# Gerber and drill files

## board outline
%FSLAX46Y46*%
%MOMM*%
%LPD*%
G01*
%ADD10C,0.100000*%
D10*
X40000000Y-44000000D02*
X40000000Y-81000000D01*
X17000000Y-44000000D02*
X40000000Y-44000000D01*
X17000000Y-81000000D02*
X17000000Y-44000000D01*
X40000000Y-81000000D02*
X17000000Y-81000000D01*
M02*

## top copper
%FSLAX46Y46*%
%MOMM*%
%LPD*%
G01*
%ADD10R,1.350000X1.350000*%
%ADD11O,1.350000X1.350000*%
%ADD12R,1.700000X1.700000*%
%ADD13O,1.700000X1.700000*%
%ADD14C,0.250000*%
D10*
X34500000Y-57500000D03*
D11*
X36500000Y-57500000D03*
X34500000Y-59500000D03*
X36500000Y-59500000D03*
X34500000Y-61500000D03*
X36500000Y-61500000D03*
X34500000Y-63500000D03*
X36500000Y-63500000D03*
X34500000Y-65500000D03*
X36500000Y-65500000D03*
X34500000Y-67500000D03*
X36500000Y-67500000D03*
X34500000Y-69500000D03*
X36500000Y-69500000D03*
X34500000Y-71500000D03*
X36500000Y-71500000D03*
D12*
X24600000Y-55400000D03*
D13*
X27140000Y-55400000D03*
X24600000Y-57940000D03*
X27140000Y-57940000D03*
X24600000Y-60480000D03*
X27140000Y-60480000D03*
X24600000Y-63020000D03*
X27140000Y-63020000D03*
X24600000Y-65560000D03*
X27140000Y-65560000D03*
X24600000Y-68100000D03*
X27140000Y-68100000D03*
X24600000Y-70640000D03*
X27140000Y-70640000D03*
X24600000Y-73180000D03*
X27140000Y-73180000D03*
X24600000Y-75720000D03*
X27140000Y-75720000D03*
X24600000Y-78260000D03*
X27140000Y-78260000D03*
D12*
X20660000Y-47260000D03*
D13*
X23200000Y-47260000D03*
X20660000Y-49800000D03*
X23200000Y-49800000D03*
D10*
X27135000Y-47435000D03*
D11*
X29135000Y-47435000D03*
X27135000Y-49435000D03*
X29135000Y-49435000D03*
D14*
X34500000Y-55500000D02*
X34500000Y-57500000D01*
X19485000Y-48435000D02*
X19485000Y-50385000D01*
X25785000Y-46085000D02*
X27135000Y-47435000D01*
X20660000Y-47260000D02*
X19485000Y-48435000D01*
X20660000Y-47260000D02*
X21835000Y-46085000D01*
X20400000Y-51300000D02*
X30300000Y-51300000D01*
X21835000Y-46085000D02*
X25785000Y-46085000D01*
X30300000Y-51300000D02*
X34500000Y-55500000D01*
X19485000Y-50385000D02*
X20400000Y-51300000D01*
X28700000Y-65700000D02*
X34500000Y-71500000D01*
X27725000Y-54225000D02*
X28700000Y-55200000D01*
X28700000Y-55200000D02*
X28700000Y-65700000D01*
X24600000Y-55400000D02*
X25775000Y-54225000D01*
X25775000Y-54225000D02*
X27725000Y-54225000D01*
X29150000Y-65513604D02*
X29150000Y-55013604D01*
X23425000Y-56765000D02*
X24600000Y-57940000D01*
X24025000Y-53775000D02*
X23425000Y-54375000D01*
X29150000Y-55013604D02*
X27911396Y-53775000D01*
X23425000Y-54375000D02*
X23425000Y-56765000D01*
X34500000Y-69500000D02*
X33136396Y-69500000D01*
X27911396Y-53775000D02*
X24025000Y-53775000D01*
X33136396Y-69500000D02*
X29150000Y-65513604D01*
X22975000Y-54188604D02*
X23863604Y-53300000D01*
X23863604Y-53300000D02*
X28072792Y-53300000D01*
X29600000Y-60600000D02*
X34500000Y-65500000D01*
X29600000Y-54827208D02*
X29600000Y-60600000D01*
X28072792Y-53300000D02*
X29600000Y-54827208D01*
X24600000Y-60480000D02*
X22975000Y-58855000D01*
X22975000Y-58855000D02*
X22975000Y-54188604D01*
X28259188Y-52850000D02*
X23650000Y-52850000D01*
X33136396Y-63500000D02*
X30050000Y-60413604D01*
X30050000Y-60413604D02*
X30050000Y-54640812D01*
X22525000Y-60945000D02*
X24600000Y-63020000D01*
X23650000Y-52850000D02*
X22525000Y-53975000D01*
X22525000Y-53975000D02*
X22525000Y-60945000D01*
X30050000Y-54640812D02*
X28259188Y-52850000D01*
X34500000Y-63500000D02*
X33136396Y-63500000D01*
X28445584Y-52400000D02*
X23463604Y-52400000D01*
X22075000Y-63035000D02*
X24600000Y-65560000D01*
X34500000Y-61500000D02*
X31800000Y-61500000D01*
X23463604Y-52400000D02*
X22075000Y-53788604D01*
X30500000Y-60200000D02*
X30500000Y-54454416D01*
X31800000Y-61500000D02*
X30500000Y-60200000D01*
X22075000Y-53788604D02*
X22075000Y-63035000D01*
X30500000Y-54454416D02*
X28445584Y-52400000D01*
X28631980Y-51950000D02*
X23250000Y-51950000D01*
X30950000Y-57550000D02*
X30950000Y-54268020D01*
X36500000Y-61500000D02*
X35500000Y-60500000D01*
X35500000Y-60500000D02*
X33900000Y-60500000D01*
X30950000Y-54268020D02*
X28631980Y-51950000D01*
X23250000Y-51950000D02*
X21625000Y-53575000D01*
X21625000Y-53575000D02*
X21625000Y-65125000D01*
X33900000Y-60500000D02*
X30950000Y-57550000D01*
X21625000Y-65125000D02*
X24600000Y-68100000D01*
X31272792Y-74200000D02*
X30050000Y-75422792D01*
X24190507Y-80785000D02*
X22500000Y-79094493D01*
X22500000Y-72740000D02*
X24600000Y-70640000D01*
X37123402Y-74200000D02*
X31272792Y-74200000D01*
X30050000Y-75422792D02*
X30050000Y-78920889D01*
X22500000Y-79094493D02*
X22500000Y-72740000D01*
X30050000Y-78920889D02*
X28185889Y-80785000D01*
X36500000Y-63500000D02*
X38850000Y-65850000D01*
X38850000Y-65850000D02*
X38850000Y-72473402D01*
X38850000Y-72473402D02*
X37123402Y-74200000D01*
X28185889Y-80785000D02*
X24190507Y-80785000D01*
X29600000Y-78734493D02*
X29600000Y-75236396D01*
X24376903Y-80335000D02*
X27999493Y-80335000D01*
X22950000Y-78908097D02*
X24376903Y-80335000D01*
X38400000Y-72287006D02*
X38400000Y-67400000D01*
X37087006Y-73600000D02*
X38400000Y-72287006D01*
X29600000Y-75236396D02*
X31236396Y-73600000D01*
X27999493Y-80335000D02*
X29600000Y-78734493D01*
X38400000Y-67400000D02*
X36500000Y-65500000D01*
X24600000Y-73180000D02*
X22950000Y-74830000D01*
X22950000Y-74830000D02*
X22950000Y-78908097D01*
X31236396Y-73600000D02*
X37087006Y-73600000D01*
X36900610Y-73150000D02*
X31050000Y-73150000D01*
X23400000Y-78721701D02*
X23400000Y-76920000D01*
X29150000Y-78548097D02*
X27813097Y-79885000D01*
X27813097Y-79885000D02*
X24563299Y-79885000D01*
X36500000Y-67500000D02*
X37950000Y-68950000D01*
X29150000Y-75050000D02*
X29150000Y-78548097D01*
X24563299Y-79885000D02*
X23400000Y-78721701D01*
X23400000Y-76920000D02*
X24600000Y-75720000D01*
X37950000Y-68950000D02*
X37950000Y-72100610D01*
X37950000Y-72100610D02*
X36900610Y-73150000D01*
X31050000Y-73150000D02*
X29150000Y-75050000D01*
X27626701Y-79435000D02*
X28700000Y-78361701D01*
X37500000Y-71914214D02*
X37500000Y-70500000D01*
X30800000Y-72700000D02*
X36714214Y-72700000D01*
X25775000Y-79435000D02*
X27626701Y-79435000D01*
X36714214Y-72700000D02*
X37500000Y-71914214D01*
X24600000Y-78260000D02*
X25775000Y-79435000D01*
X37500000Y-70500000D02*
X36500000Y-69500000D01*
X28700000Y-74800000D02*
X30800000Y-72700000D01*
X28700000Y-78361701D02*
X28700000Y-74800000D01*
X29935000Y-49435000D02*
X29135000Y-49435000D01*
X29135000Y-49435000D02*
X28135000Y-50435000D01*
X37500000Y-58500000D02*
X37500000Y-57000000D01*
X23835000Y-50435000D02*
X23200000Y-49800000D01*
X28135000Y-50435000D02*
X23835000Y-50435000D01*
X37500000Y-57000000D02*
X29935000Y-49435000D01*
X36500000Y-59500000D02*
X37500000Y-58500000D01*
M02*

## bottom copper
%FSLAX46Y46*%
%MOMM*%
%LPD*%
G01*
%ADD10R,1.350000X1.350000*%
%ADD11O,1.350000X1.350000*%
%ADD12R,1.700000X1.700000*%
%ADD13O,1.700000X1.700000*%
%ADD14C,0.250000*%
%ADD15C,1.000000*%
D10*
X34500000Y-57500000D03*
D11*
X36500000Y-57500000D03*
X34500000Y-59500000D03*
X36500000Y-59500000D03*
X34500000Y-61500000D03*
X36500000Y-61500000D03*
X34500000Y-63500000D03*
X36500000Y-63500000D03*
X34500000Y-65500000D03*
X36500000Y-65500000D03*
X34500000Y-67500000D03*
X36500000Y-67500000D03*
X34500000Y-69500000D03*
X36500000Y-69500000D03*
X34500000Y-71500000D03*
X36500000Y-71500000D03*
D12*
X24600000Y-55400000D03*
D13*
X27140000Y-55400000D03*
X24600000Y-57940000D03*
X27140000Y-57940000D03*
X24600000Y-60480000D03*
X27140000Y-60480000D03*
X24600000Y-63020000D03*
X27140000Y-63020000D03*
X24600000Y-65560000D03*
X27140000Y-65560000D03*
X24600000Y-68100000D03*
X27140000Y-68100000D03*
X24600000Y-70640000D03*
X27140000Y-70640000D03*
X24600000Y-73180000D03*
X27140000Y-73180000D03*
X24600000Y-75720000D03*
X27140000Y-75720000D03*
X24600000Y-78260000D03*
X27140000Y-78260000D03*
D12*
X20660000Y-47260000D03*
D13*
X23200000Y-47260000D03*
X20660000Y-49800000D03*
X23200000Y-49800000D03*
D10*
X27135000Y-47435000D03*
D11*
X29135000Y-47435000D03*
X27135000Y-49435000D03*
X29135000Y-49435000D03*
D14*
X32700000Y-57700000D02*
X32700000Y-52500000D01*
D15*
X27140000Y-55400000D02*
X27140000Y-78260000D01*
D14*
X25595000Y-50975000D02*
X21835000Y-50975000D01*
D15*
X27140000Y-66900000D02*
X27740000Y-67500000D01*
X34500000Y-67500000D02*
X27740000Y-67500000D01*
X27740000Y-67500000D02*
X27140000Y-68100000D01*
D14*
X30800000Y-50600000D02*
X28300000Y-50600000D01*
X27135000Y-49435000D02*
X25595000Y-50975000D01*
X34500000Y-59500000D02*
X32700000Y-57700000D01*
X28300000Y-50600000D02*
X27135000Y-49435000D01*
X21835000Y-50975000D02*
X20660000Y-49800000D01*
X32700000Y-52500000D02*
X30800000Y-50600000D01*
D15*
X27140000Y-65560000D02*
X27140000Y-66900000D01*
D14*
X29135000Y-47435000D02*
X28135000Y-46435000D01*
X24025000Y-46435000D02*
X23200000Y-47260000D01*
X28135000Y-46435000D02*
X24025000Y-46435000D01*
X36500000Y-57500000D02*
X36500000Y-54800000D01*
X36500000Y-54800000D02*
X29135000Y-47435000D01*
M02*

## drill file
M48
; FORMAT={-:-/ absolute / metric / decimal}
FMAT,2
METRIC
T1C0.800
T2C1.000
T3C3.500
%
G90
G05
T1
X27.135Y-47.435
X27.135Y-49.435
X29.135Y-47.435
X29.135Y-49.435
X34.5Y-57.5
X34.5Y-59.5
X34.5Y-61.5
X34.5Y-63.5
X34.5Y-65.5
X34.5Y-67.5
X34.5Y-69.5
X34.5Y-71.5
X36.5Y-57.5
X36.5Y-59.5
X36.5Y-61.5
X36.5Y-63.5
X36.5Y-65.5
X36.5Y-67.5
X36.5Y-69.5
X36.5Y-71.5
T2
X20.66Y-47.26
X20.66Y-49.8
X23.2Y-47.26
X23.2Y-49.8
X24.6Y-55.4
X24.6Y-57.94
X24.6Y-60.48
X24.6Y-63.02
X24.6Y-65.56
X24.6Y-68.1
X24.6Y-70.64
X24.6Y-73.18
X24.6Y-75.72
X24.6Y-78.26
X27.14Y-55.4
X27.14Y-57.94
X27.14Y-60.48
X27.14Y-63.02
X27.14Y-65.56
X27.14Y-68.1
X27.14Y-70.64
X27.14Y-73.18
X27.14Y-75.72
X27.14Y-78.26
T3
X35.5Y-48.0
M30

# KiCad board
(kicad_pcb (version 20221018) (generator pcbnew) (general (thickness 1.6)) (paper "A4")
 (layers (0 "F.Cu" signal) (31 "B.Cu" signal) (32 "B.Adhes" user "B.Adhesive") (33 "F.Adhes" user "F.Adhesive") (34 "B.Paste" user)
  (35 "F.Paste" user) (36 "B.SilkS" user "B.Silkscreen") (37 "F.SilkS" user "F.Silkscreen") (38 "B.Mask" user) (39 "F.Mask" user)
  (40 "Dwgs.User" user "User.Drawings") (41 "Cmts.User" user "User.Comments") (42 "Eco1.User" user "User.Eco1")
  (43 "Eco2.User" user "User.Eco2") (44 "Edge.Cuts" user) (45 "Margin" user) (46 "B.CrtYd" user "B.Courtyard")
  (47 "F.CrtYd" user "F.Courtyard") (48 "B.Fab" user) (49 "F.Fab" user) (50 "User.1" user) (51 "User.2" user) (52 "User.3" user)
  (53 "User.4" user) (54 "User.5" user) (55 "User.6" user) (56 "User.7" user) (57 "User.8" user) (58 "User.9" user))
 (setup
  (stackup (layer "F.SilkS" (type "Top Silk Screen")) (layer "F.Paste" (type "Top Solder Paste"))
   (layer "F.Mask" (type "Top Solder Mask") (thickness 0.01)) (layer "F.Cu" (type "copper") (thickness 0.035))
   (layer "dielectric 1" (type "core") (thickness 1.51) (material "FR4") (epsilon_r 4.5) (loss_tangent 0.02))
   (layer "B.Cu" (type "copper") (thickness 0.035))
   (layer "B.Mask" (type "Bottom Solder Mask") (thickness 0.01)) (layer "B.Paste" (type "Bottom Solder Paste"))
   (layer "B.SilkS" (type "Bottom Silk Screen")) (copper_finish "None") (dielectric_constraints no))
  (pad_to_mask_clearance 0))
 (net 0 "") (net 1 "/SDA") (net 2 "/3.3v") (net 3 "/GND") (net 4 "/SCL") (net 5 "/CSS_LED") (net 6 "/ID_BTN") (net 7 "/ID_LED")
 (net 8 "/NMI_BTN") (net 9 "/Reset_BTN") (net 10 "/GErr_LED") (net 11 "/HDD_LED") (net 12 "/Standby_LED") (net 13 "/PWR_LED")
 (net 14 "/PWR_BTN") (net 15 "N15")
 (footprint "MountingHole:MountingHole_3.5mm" (layer "F.Cu") (at 35.5 48)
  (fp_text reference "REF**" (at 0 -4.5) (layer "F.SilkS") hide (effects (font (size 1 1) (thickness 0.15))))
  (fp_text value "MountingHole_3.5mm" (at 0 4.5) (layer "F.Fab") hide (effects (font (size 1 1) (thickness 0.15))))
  (pad "" np_thru_hole circle (at 0 0) (size 3.5 3.5) (drill 3.5) (layers "*.Cu" "*.Mask")))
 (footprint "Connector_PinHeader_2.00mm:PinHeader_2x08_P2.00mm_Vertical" (layer "F.Cu") (at 34.5 57.5)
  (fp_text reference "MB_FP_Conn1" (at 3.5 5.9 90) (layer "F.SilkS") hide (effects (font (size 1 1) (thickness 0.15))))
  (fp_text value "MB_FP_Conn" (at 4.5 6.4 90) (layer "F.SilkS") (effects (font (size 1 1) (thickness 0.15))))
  (pad "1" thru_hole rect (at 0 0) (size 1.35 1.35) (drill 0.8) (layers "*.Cu" "*.Mask") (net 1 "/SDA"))
  (pad "2" thru_hole oval (at 2 0) (size 1.35 1.35) (drill 0.8) (layers "*.Cu" "*.Mask") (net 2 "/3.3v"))
  (pad "3" thru_hole oval (at 0 2) (size 1.35 1.35) (drill 0.8) (layers "*.Cu" "*.Mask") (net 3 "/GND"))
  (pad "4" thru_hole oval (at 2 2) (size 1.35 1.35) (drill 0.8) (layers "*.Cu" "*.Mask") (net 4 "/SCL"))
  (pad "5" thru_hole oval (at 0 4) (size 1.35 1.35) (drill 0.8) (layers "*.Cu" "*.Mask") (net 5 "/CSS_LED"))
  (pad "6" thru_hole oval (at 2 4) (size 1.35 1.35) (drill 0.8) (layers "*.Cu" "*.Mask") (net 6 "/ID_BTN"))
  (pad "7" thru_hole oval (at 0 6) (size 1.35 1.35) (drill 0.8) (layers "*.Cu" "*.Mask") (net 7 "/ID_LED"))
  (pad "8" thru_hole oval (at 2 6) (size 1.35 1.35) (drill 0.8) (layers "*.Cu" "*.Mask") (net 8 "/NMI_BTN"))
  (pad "9" thru_hole oval (at 0 8) (size 1.35 1.35) (drill 0.8) (layers "*.Cu" "*.Mask") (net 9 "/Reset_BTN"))
  (pad "10" thru_hole oval (at 2 8) (size 1.35 1.35) (drill 0.8) (layers "*.Cu" "*.Mask") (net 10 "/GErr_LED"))
  (pad "11" thru_hole oval (at 0 10) (size 1.35 1.35) (drill 0.8) (layers "*.Cu" "*.Mask") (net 3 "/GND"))
  (pad "12" thru_hole oval (at 2 10) (size 1.35 1.35) (drill 0.8) (layers "*.Cu" "*.Mask") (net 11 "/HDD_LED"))
  (pad "13" thru_hole oval (at 0 12) (size 1.35 1.35) (drill 0.8) (layers "*.Cu" "*.Mask") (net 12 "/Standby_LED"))
  (pad "14" thru_hole oval (at 2 12) (size 1.35 1.35) (drill 0.8) (layers "*.Cu" "*.Mask") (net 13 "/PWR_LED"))
  (pad "15" thru_hole oval (at 0 14) (size 1.35 1.35) (drill 0.8) (layers "*.Cu" "*.Mask") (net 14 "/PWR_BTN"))
  (pad "16" thru_hole oval (at 2 14) (size 1.35 1.35) (drill 0.8) (layers "*.Cu" "*.Mask") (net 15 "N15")))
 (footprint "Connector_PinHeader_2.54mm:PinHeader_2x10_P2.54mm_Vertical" (layer "F.Cu") (at 24.6 55.4)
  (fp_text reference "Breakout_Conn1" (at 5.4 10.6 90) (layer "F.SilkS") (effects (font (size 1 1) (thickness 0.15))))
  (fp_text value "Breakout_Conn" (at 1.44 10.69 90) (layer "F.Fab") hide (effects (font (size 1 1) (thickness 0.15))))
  (pad "1" thru_hole rect (at 0 0) (size 1.7 1.7) (drill 1) (layers "*.Cu" "*.Mask") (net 14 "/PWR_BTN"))
  (pad "2" thru_hole oval (at 2.54 0) (size 1.7 1.7) (drill 1) (layers "*.Cu" "*.Mask") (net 3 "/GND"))
  (pad "3" thru_hole oval (at 0 2.54) (size 1.7 1.7) (drill 1) (layers "*.Cu" "*.Mask") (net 12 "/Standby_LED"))
  (pad "4" thru_hole oval (at 2.54 2.54) (size 1.7 1.7) (drill 1) (layers "*.Cu" "*.Mask") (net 3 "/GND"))
  (pad "5" thru_hole oval (at 0 5.08) (size 1.7 1.7) (drill 1) (layers "*.Cu" "*.Mask") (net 9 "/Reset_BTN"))
  (pad "6" thru_hole oval (at 2.54 5.08) (size 1.7 1.7) (drill 1) (layers "*.Cu" "*.Mask") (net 3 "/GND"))
  (pad "7" thru_hole oval (at 0 7.62) (size 1.7 1.7) (drill 1) (layers "*.Cu" "*.Mask") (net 7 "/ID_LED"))
  (pad "8" thru_hole oval (at 2.54 7.62) (size 1.7 1.7) (drill 1) (layers "*.Cu" "*.Mask") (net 3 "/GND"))
  (pad "9" thru_hole oval (at 0 10.16) (size 1.7 1.7) (drill 1) (layers "*.Cu" "*.Mask") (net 5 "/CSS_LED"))
  (pad "10" thru_hole oval (at 2.54 10.16) (size 1.7 1.7) (drill 1) (layers "*.Cu" "*.Mask") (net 3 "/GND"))
  (pad "11" thru_hole oval (at 0 12.7) (size 1.7 1.7) (drill 1) (layers "*.Cu" "*.Mask") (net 6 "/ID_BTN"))
  (pad "12" thru_hole oval (at 2.54 12.7) (size 1.7 1.7) (drill 1) (layers "*.Cu" "*.Mask") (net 3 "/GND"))
  (pad "13" thru_hole oval (at 0 15.24) (size 1.7 1.7) (drill 1) (layers "*.Cu" "*.Mask") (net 8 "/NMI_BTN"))
  (pad "14" thru_hole oval (at 2.54 15.24) (size 1.7 1.7) (drill 1) (layers "*.Cu" "*.Mask") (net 3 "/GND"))
  (pad "15" thru_hole oval (at 0 17.78) (size 1.7 1.7) (drill 1) (layers "*.Cu" "*.Mask") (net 10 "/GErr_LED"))
  (pad "16" thru_hole oval (at 2.54 17.78) (size 1.7 1.7) (drill 1) (layers "*.Cu" "*.Mask") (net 3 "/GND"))
  (pad "17" thru_hole oval (at 0 20.32) (size 1.7 1.7) (drill 1) (layers "*.Cu" "*.Mask") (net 11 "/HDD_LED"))
  (pad "18" thru_hole oval (at 2.54 20.32) (size 1.7 1.7) (drill 1) (layers "*.Cu" "*.Mask") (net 3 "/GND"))
  (pad "19" thru_hole oval (at 0 22.86) (size 1.7 1.7) (drill 1) (layers "*.Cu" "*.Mask") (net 13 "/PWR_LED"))
  (pad "20" thru_hole oval (at 2.54 22.86) (size 1.7 1.7) (drill 1) (layers "*.Cu" "*.Mask") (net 3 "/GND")))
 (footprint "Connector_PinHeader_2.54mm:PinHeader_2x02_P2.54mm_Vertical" (layer "F.Cu") (at 20.66 47.26)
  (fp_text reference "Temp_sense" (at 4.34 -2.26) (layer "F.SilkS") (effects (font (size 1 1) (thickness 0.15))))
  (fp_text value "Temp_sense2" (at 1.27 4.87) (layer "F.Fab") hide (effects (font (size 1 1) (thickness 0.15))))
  (pad "1" thru_hole rect (at 0 0) (size 1.7 1.7) (drill 1) (layers "*.Cu" "*.Mask") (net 1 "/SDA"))
  (pad "2" thru_hole oval (at 2.54 0) (size 1.7 1.7) (drill 1) (layers "*.Cu" "*.Mask") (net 2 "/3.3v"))
  (pad "3" thru_hole oval (at 0 2.54) (size 1.7 1.7) (drill 1) (layers "*.Cu" "*.Mask") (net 3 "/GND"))
  (pad "4" thru_hole oval (at 2.54 2.54) (size 1.7 1.7) (drill 1) (layers "*.Cu" "*.Mask") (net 4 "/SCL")))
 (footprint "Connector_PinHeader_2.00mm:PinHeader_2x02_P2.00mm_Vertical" (layer "F.Cu") (at 27.135 47.435)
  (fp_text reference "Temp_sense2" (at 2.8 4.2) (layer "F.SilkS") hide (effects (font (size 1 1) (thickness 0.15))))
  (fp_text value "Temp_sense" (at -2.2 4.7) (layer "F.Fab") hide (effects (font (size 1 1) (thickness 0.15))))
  (pad "1" thru_hole rect (at 0 0) (size 1.35 1.35) (drill 0.8) (layers "*.Cu" "*.Mask") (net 1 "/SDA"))
  (pad "2" thru_hole oval (at 2 0) (size 1.35 1.35) (drill 0.8) (layers "*.Cu" "*.Mask") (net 2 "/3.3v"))
  (pad "3" thru_hole oval (at 0 2) (size 1.35 1.35) (drill 0.8) (layers "*.Cu" "*.Mask") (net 3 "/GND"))
  (pad "4" thru_hole oval (at 2 2) (size 1.35 1.35) (drill 0.8) (layers "*.Cu" "*.Mask") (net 4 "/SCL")))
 (gr_line (start 40 44) (end 40 81) (stroke (width 0.1) (type default)) (layer "Edge.Cuts"))
 (gr_line (start 17 44) (end 40 44) (stroke (width 0.1) (type default)) (layer "Edge.Cuts"))
 (gr_line (start 17 81) (end 17 44) (stroke (width 0.1) (type default)) (layer "Edge.Cuts"))
 (gr_line (start 40 81) (end 17 81) (stroke (width 0.1) (type default)) (layer "Edge.Cuts"))
 (segment (start 34.5 55.5) (end 34.5 57.5) (width 0.25) (layer "F.Cu") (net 1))
 (segment (start 19.485 48.435) (end 19.485 50.385) (width 0.25) (layer "F.Cu") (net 1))
 (segment (start 25.785 46.085) (end 27.135 47.435) (width 0.25) (layer "F.Cu") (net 1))
 (segment (start 20.66 47.26) (end 19.485 48.435) (width 0.25) (layer "F.Cu") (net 1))
 (segment (start 20.66 47.26) (end 21.835 46.085) (width 0.25) (layer "F.Cu") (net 1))
 (segment (start 20.4 51.3) (end 30.3 51.3) (width 0.25) (layer "F.Cu") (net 1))
 (segment (start 21.835 46.085) (end 25.785 46.085) (width 0.25) (layer "F.Cu") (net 1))
 (segment (start 30.3 51.3) (end 34.5 55.5) (width 0.25) (layer "F.Cu") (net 1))
 (segment (start 19.485 50.385) (end 20.4 51.3) (width 0.25) (layer "F.Cu") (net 1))
 (segment (start 28.7 65.7) (end 34.5 71.5) (width 0.25) (layer "F.Cu") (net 14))
 (segment (start 27.725 54.225) (end 28.7 55.2) (width 0.25) (layer "F.Cu") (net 14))
 (segment (start 28.7 55.2) (end 28.7 65.7) (width 0.25) (layer "F.Cu") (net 14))
 (segment (start 24.6 55.4) (end 25.775 54.225) (width 0.25) (layer "F.Cu") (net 14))
 (segment (start 25.775 54.225) (end 27.725 54.225) (width 0.25) (layer "F.Cu") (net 14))
 (segment (start 32.7 57.7) (end 32.7 52.5) (width 0.25) (layer "B.Cu") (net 3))
 (segment (start 27.14 55.4) (end 27.14 78.26) (width 1) (layer "B.Cu") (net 3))
 (segment (start 25.595 50.975) (end 21.835 50.975) (width 0.25) (layer "B.Cu") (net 3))
 (segment (start 27.14 66.9) (end 27.74 67.5) (width 1) (layer "B.Cu") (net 3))
 (segment (start 34.5 67.5) (end 27.74 67.5) (width 1) (layer "B.Cu") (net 3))
 (segment (start 27.74 67.5) (end 27.14 68.1) (width 1) (layer "B.Cu") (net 3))
 (segment (start 30.8 50.6) (end 28.3 50.6) (width 0.25) (layer "B.Cu") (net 3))
 (segment (start 27.135 49.435) (end 25.595 50.975) (width 0.25) (layer "B.Cu") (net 3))
 (segment (start 34.5 59.5) (end 32.7 57.7) (width 0.25) (layer "B.Cu") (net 3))
 (segment (start 28.3 50.6) (end 27.135 49.435) (width 0.25) (layer "B.Cu") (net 3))
 (segment (start 21.835 50.975) (end 20.66 49.8) (width 0.25) (layer "B.Cu") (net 3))
 (segment (start 32.7 52.5) (end 30.8 50.6) (width 0.25) (layer "B.Cu") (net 3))
 (segment (start 27.14 65.56) (end 27.14 66.9) (width 1) (layer "B.Cu") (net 3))
 (segment (start 29.15 65.513604) (end 29.15 55.013604) (width 0.25) (layer "F.Cu") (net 12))
 (segment (start 23.425 56.765) (end 24.6 57.94) (width 0.25) (layer "F.Cu") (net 12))
 (segment (start 24.025 53.775) (end 23.425 54.375) (width 0.25) (layer "F.Cu") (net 12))
 (segment (start 29.15 55.013604) (end 27.911396 53.775) (width 0.25) (layer "F.Cu") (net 12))
 (segment (start 23.425 54.375) (end 23.425 56.765) (width 0.25) (layer "F.Cu") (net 12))
 (segment (start 34.5 69.5) (end 33.136396 69.5) (width 0.25) (layer "F.Cu") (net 12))
 (segment (start 27.911396 53.775) (end 24.025 53.775) (width 0.25) (layer "F.Cu") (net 12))
 (segment (start 33.136396 69.5) (end 29.15 65.513604) (width 0.25) (layer "F.Cu") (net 12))
 (segment (start 22.975 54.188604) (end 23.863604 53.3) (width 0.25) (layer "F.Cu") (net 9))
 (segment (start 23.863604 53.3) (end 28.072792 53.3) (width 0.25) (layer "F.Cu") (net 9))
 (segment (start 29.6 60.6) (end 34.5 65.5) (width 0.25) (layer "F.Cu") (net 9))
 (segment (start 29.6 54.827208) (end 29.6 60.6) (width 0.25) (layer "F.Cu") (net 9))
 (segment (start 28.072792 53.3) (end 29.6 54.827208) (width 0.25) (layer "F.Cu") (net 9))
 (segment (start 24.6 60.48) (end 22.975 58.855) (width 0.25) (layer "F.Cu") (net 9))
 (segment (start 22.975 58.855) (end 22.975 54.188604) (width 0.25) (layer "F.Cu") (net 9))
 (segment (start 28.259188 52.85) (end 23.65 52.85) (width 0.25) (layer "F.Cu") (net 7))
 (segment (start 33.136396 63.5) (end 30.05 60.413604) (width 0.25) (layer "F.Cu") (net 7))
 (segment (start 30.05 60.413604) (end 30.05 54.640812) (width 0.25) (layer "F.Cu") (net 7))
 (segment (start 22.525 60.945) (end 24.6 63.02) (width 0.25) (layer "F.Cu") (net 7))
 (segment (start 23.65 52.85) (end 22.525 53.975) (width 0.25) (layer "F.Cu") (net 7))
 (segment (start 22.525 53.975) (end 22.525 60.945) (width 0.25) (layer "F.Cu") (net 7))
 (segment (start 30.05 54.640812) (end 28.259188 52.85) (width 0.25) (layer "F.Cu") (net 7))
 (segment (start 34.5 63.5) (end 33.136396 63.5) (width 0.25) (layer "F.Cu") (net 7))
 (segment (start 28.445584 52.4) (end 23.463604 52.4) (width 0.25) (layer "F.Cu") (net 5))
 (segment (start 22.075 63.035) (end 24.6 65.56) (width 0.25) (layer "F.Cu") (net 5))
 (segment (start 34.5 61.5) (end 31.8 61.5) (width 0.25) (layer "F.Cu") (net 5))
 (segment (start 23.463604 52.4) (end 22.075 53.788604) (width 0.25) (layer "F.Cu") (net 5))
 (segment (start 30.5 60.2) (end 30.5 54.454416) (width 0.25) (layer "F.Cu") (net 5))
 (segment (start 31.8 61.5) (end 30.5 60.2) (width 0.25) (layer "F.Cu") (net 5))
 (segment (start 22.075 53.788604) (end 22.075 63.035) (width 0.25) (layer "F.Cu") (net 5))
 (segment (start 30.5 54.454416) (end 28.445584 52.4) (width 0.25) (layer "F.Cu") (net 5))
 (segment (start 28.63198 51.95) (end 23.25 51.95) (width 0.25) (layer "F.Cu") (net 6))
 (segment (start 30.95 57.55) (end 30.95 54.26802) (width 0.25) (layer "F.Cu") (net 6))
 (segment (start 36.5 61.5) (end 35.5 60.5) (width 0.25) (layer "F.Cu") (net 6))
 (segment (start 35.5 60.5) (end 33.9 60.5) (width 0.25) (layer "F.Cu") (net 6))
 (segment (start 30.95 54.26802) (end 28.63198 51.95) (width 0.25) (layer "F.Cu") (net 6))
 (segment (start 23.25 51.95) (end 21.625 53.575) (width 0.25) (layer "F.Cu") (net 6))
 (segment (start 21.625 53.575) (end 21.625 65.125) (width 0.25) (layer "F.Cu") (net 6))
 (segment (start 33.9 60.5) (end 30.95 57.55) (width 0.25) (layer "F.Cu") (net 6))
 (segment (start 21.625 65.125) (end 24.6 68.1) (width 0.25) (layer "F.Cu") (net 6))
 (segment (start 31.272792 74.2) (end 30.05 75.422792) (width 0.25) (layer "F.Cu") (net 8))
 (segment (start 24.190507 80.785) (end 22.5 79.094493) (width 0.25) (layer "F.Cu") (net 8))
 (segment (start 22.5 72.74) (end 24.6 70.64) (width 0.25) (layer "F.Cu") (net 8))
 (segment (start 37.123402 74.2) (end 31.272792 74.2) (width 0.25) (layer "F.Cu") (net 8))
 (segment (start 30.05 75.422792) (end 30.05 78.920889) (width 0.25) (layer "F.Cu") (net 8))
 (segment (start 22.5 79.094493) (end 22.5 72.74) (width 0.25) (layer "F.Cu") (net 8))
 (segment (start 30.05 78.920889) (end 28.185889 80.785) (width 0.25) (layer "F.Cu") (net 8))
 (segment (start 36.5 63.5) (end 38.85 65.85) (width 0.25) (layer "F.Cu") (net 8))
 (segment (start 38.85 65.85) (end 38.85 72.473402) (width 0.25) (layer "F.Cu") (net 8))
 (segment (start 38.85 72.473402) (end 37.123402 74.2) (width 0.25) (layer "F.Cu") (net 8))
 (segment (start 28.185889 80.785) (end 24.190507 80.785) (width 0.25) (layer "F.Cu") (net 8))
 (segment (start 29.6 78.734493) (end 29.6 75.236396) (width 0.25) (layer "F.Cu") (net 10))
 (segment (start 24.376903 80.335) (end 27.999493 80.335) (width 0.25) (layer "F.Cu") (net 10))
 (segment (start 22.95 78.908097) (end 24.376903 80.335) (width 0.25) (layer "F.Cu") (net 10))
 (segment (start 38.4 72.287006) (end 38.4 67.4) (width 0.25) (layer "F.Cu") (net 10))
 (segment (start 37.087006 73.6) (end 38.4 72.287006) (width 0.25) (layer "F.Cu") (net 10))
 (segment (start 29.6 75.236396) (end 31.236396 73.6) (width 0.25) (layer "F.Cu") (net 10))
 (segment (start 27.999493 80.335) (end 29.6 78.734493) (width 0.25) (layer "F.Cu") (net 10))
 (segment (start 38.4 67.4) (end 36.5 65.5) (width 0.25) (layer "F.Cu") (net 10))
 (segment (start 24.6 73.18) (end 22.95 74.83) (width 0.25) (layer "F.Cu") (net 10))
 (segment (start 22.95 74.83) (end 22.95 78.908097) (width 0.25) (layer "F.Cu") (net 10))
 (segment (start 31.236396 73.6) (end 37.087006 73.6) (width 0.25) (layer "F.Cu") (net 10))
 (segment (start 36.90061 73.15) (end 31.05 73.15) (width 0.25) (layer "F.Cu") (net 11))
 (segment (start 23.4 78.721701) (end 23.4 76.92) (width 0.25) (layer "F.Cu") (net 11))
 (segment (start 29.15 78.548097) (end 27.813097 79.885) (width 0.25) (layer "F.Cu") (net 11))
 (segment (start 27.813097 79.885) (end 24.563299 79.885) (width 0.25) (layer "F.Cu") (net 11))
 (segment (start 36.5 67.5) (end 37.95 68.95) (width 0.25) (layer "F.Cu") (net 11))
 (segment (start 29.15 75.05) (end 29.15 78.548097) (width 0.25) (layer "F.Cu") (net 11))
 (segment (start 24.563299 79.885) (end 23.4 78.721701) (width 0.25) (layer "F.Cu") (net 11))
 (segment (start 23.4 76.92) (end 24.6 75.72) (width 0.25) (layer "F.Cu") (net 11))
 (segment (start 37.95 68.95) (end 37.95 72.10061) (width 0.25) (layer "F.Cu") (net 11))
 (segment (start 37.95 72.10061) (end 36.90061 73.15) (width 0.25) (layer "F.Cu") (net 11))
 (segment (start 31.05 73.15) (end 29.15 75.05) (width 0.25) (layer "F.Cu") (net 11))
 (segment (start 27.626701 79.435) (end 28.7 78.361701) (width 0.25) (layer "F.Cu") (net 13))
 (segment (start 37.5 71.914214) (end 37.5 70.5) (width 0.25) (layer "F.Cu") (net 13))
 (segment (start 30.8 72.7) (end 36.714214 72.7) (width 0.25) (layer "F.Cu") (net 13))
 (segment (start 25.775 79.435) (end 27.626701 79.435) (width 0.25) (layer "F.Cu") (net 13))
 (segment (start 36.714214 72.7) (end 37.5 71.914214) (width 0.25) (layer "F.Cu") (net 13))
 (segment (start 24.6 78.26) (end 25.775 79.435) (width 0.25) (layer "F.Cu") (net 13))
 (segment (start 37.5 70.5) (end 36.5 69.5) (width 0.25) (layer "F.Cu") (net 13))
 (segment (start 28.7 74.8) (end 30.8 72.7) (width 0.25) (layer "F.Cu") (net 13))
 (segment (start 28.7 78.361701) (end 28.7 74.8) (width 0.25) (layer "F.Cu") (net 13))
 (segment (start 29.135 47.435) (end 28.135 46.435) (width 0.25) (layer "B.Cu") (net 2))
 (segment (start 24.025 46.435) (end 23.2 47.26) (width 0.25) (layer "B.Cu") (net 2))
 (segment (start 28.135 46.435) (end 24.025 46.435) (width 0.25) (layer "B.Cu") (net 2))
 (segment (start 36.5 57.5) (end 36.5 54.8) (width 0.25) (layer "B.Cu") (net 2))
 (segment (start 36.5 54.8) (end 29.135 47.435) (width 0.25) (layer "B.Cu") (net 2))
 (segment (start 29.935 49.435) (end 29.135 49.435) (width 0.25) (layer "F.Cu") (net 4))
 (segment (start 29.135 49.435) (end 28.135 50.435) (width 0.25) (layer "F.Cu") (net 4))
 (segment (start 37.5 58.5) (end 37.5 57) (width 0.25) (layer "F.Cu") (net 4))
 (segment (start 23.835 50.435) (end 23.2 49.8) (width 0.25) (layer "F.Cu") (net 4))
 (segment (start 28.135 50.435) (end 23.835 50.435) (width 0.25) (layer "F.Cu") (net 4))
 (segment (start 37.5 57) (end 29.935 49.435) (width 0.25) (layer "F.Cu") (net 4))
 (segment (start 36.5 59.5) (end 37.5 58.5) (width 0.25) (layer "F.Cu") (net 4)))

